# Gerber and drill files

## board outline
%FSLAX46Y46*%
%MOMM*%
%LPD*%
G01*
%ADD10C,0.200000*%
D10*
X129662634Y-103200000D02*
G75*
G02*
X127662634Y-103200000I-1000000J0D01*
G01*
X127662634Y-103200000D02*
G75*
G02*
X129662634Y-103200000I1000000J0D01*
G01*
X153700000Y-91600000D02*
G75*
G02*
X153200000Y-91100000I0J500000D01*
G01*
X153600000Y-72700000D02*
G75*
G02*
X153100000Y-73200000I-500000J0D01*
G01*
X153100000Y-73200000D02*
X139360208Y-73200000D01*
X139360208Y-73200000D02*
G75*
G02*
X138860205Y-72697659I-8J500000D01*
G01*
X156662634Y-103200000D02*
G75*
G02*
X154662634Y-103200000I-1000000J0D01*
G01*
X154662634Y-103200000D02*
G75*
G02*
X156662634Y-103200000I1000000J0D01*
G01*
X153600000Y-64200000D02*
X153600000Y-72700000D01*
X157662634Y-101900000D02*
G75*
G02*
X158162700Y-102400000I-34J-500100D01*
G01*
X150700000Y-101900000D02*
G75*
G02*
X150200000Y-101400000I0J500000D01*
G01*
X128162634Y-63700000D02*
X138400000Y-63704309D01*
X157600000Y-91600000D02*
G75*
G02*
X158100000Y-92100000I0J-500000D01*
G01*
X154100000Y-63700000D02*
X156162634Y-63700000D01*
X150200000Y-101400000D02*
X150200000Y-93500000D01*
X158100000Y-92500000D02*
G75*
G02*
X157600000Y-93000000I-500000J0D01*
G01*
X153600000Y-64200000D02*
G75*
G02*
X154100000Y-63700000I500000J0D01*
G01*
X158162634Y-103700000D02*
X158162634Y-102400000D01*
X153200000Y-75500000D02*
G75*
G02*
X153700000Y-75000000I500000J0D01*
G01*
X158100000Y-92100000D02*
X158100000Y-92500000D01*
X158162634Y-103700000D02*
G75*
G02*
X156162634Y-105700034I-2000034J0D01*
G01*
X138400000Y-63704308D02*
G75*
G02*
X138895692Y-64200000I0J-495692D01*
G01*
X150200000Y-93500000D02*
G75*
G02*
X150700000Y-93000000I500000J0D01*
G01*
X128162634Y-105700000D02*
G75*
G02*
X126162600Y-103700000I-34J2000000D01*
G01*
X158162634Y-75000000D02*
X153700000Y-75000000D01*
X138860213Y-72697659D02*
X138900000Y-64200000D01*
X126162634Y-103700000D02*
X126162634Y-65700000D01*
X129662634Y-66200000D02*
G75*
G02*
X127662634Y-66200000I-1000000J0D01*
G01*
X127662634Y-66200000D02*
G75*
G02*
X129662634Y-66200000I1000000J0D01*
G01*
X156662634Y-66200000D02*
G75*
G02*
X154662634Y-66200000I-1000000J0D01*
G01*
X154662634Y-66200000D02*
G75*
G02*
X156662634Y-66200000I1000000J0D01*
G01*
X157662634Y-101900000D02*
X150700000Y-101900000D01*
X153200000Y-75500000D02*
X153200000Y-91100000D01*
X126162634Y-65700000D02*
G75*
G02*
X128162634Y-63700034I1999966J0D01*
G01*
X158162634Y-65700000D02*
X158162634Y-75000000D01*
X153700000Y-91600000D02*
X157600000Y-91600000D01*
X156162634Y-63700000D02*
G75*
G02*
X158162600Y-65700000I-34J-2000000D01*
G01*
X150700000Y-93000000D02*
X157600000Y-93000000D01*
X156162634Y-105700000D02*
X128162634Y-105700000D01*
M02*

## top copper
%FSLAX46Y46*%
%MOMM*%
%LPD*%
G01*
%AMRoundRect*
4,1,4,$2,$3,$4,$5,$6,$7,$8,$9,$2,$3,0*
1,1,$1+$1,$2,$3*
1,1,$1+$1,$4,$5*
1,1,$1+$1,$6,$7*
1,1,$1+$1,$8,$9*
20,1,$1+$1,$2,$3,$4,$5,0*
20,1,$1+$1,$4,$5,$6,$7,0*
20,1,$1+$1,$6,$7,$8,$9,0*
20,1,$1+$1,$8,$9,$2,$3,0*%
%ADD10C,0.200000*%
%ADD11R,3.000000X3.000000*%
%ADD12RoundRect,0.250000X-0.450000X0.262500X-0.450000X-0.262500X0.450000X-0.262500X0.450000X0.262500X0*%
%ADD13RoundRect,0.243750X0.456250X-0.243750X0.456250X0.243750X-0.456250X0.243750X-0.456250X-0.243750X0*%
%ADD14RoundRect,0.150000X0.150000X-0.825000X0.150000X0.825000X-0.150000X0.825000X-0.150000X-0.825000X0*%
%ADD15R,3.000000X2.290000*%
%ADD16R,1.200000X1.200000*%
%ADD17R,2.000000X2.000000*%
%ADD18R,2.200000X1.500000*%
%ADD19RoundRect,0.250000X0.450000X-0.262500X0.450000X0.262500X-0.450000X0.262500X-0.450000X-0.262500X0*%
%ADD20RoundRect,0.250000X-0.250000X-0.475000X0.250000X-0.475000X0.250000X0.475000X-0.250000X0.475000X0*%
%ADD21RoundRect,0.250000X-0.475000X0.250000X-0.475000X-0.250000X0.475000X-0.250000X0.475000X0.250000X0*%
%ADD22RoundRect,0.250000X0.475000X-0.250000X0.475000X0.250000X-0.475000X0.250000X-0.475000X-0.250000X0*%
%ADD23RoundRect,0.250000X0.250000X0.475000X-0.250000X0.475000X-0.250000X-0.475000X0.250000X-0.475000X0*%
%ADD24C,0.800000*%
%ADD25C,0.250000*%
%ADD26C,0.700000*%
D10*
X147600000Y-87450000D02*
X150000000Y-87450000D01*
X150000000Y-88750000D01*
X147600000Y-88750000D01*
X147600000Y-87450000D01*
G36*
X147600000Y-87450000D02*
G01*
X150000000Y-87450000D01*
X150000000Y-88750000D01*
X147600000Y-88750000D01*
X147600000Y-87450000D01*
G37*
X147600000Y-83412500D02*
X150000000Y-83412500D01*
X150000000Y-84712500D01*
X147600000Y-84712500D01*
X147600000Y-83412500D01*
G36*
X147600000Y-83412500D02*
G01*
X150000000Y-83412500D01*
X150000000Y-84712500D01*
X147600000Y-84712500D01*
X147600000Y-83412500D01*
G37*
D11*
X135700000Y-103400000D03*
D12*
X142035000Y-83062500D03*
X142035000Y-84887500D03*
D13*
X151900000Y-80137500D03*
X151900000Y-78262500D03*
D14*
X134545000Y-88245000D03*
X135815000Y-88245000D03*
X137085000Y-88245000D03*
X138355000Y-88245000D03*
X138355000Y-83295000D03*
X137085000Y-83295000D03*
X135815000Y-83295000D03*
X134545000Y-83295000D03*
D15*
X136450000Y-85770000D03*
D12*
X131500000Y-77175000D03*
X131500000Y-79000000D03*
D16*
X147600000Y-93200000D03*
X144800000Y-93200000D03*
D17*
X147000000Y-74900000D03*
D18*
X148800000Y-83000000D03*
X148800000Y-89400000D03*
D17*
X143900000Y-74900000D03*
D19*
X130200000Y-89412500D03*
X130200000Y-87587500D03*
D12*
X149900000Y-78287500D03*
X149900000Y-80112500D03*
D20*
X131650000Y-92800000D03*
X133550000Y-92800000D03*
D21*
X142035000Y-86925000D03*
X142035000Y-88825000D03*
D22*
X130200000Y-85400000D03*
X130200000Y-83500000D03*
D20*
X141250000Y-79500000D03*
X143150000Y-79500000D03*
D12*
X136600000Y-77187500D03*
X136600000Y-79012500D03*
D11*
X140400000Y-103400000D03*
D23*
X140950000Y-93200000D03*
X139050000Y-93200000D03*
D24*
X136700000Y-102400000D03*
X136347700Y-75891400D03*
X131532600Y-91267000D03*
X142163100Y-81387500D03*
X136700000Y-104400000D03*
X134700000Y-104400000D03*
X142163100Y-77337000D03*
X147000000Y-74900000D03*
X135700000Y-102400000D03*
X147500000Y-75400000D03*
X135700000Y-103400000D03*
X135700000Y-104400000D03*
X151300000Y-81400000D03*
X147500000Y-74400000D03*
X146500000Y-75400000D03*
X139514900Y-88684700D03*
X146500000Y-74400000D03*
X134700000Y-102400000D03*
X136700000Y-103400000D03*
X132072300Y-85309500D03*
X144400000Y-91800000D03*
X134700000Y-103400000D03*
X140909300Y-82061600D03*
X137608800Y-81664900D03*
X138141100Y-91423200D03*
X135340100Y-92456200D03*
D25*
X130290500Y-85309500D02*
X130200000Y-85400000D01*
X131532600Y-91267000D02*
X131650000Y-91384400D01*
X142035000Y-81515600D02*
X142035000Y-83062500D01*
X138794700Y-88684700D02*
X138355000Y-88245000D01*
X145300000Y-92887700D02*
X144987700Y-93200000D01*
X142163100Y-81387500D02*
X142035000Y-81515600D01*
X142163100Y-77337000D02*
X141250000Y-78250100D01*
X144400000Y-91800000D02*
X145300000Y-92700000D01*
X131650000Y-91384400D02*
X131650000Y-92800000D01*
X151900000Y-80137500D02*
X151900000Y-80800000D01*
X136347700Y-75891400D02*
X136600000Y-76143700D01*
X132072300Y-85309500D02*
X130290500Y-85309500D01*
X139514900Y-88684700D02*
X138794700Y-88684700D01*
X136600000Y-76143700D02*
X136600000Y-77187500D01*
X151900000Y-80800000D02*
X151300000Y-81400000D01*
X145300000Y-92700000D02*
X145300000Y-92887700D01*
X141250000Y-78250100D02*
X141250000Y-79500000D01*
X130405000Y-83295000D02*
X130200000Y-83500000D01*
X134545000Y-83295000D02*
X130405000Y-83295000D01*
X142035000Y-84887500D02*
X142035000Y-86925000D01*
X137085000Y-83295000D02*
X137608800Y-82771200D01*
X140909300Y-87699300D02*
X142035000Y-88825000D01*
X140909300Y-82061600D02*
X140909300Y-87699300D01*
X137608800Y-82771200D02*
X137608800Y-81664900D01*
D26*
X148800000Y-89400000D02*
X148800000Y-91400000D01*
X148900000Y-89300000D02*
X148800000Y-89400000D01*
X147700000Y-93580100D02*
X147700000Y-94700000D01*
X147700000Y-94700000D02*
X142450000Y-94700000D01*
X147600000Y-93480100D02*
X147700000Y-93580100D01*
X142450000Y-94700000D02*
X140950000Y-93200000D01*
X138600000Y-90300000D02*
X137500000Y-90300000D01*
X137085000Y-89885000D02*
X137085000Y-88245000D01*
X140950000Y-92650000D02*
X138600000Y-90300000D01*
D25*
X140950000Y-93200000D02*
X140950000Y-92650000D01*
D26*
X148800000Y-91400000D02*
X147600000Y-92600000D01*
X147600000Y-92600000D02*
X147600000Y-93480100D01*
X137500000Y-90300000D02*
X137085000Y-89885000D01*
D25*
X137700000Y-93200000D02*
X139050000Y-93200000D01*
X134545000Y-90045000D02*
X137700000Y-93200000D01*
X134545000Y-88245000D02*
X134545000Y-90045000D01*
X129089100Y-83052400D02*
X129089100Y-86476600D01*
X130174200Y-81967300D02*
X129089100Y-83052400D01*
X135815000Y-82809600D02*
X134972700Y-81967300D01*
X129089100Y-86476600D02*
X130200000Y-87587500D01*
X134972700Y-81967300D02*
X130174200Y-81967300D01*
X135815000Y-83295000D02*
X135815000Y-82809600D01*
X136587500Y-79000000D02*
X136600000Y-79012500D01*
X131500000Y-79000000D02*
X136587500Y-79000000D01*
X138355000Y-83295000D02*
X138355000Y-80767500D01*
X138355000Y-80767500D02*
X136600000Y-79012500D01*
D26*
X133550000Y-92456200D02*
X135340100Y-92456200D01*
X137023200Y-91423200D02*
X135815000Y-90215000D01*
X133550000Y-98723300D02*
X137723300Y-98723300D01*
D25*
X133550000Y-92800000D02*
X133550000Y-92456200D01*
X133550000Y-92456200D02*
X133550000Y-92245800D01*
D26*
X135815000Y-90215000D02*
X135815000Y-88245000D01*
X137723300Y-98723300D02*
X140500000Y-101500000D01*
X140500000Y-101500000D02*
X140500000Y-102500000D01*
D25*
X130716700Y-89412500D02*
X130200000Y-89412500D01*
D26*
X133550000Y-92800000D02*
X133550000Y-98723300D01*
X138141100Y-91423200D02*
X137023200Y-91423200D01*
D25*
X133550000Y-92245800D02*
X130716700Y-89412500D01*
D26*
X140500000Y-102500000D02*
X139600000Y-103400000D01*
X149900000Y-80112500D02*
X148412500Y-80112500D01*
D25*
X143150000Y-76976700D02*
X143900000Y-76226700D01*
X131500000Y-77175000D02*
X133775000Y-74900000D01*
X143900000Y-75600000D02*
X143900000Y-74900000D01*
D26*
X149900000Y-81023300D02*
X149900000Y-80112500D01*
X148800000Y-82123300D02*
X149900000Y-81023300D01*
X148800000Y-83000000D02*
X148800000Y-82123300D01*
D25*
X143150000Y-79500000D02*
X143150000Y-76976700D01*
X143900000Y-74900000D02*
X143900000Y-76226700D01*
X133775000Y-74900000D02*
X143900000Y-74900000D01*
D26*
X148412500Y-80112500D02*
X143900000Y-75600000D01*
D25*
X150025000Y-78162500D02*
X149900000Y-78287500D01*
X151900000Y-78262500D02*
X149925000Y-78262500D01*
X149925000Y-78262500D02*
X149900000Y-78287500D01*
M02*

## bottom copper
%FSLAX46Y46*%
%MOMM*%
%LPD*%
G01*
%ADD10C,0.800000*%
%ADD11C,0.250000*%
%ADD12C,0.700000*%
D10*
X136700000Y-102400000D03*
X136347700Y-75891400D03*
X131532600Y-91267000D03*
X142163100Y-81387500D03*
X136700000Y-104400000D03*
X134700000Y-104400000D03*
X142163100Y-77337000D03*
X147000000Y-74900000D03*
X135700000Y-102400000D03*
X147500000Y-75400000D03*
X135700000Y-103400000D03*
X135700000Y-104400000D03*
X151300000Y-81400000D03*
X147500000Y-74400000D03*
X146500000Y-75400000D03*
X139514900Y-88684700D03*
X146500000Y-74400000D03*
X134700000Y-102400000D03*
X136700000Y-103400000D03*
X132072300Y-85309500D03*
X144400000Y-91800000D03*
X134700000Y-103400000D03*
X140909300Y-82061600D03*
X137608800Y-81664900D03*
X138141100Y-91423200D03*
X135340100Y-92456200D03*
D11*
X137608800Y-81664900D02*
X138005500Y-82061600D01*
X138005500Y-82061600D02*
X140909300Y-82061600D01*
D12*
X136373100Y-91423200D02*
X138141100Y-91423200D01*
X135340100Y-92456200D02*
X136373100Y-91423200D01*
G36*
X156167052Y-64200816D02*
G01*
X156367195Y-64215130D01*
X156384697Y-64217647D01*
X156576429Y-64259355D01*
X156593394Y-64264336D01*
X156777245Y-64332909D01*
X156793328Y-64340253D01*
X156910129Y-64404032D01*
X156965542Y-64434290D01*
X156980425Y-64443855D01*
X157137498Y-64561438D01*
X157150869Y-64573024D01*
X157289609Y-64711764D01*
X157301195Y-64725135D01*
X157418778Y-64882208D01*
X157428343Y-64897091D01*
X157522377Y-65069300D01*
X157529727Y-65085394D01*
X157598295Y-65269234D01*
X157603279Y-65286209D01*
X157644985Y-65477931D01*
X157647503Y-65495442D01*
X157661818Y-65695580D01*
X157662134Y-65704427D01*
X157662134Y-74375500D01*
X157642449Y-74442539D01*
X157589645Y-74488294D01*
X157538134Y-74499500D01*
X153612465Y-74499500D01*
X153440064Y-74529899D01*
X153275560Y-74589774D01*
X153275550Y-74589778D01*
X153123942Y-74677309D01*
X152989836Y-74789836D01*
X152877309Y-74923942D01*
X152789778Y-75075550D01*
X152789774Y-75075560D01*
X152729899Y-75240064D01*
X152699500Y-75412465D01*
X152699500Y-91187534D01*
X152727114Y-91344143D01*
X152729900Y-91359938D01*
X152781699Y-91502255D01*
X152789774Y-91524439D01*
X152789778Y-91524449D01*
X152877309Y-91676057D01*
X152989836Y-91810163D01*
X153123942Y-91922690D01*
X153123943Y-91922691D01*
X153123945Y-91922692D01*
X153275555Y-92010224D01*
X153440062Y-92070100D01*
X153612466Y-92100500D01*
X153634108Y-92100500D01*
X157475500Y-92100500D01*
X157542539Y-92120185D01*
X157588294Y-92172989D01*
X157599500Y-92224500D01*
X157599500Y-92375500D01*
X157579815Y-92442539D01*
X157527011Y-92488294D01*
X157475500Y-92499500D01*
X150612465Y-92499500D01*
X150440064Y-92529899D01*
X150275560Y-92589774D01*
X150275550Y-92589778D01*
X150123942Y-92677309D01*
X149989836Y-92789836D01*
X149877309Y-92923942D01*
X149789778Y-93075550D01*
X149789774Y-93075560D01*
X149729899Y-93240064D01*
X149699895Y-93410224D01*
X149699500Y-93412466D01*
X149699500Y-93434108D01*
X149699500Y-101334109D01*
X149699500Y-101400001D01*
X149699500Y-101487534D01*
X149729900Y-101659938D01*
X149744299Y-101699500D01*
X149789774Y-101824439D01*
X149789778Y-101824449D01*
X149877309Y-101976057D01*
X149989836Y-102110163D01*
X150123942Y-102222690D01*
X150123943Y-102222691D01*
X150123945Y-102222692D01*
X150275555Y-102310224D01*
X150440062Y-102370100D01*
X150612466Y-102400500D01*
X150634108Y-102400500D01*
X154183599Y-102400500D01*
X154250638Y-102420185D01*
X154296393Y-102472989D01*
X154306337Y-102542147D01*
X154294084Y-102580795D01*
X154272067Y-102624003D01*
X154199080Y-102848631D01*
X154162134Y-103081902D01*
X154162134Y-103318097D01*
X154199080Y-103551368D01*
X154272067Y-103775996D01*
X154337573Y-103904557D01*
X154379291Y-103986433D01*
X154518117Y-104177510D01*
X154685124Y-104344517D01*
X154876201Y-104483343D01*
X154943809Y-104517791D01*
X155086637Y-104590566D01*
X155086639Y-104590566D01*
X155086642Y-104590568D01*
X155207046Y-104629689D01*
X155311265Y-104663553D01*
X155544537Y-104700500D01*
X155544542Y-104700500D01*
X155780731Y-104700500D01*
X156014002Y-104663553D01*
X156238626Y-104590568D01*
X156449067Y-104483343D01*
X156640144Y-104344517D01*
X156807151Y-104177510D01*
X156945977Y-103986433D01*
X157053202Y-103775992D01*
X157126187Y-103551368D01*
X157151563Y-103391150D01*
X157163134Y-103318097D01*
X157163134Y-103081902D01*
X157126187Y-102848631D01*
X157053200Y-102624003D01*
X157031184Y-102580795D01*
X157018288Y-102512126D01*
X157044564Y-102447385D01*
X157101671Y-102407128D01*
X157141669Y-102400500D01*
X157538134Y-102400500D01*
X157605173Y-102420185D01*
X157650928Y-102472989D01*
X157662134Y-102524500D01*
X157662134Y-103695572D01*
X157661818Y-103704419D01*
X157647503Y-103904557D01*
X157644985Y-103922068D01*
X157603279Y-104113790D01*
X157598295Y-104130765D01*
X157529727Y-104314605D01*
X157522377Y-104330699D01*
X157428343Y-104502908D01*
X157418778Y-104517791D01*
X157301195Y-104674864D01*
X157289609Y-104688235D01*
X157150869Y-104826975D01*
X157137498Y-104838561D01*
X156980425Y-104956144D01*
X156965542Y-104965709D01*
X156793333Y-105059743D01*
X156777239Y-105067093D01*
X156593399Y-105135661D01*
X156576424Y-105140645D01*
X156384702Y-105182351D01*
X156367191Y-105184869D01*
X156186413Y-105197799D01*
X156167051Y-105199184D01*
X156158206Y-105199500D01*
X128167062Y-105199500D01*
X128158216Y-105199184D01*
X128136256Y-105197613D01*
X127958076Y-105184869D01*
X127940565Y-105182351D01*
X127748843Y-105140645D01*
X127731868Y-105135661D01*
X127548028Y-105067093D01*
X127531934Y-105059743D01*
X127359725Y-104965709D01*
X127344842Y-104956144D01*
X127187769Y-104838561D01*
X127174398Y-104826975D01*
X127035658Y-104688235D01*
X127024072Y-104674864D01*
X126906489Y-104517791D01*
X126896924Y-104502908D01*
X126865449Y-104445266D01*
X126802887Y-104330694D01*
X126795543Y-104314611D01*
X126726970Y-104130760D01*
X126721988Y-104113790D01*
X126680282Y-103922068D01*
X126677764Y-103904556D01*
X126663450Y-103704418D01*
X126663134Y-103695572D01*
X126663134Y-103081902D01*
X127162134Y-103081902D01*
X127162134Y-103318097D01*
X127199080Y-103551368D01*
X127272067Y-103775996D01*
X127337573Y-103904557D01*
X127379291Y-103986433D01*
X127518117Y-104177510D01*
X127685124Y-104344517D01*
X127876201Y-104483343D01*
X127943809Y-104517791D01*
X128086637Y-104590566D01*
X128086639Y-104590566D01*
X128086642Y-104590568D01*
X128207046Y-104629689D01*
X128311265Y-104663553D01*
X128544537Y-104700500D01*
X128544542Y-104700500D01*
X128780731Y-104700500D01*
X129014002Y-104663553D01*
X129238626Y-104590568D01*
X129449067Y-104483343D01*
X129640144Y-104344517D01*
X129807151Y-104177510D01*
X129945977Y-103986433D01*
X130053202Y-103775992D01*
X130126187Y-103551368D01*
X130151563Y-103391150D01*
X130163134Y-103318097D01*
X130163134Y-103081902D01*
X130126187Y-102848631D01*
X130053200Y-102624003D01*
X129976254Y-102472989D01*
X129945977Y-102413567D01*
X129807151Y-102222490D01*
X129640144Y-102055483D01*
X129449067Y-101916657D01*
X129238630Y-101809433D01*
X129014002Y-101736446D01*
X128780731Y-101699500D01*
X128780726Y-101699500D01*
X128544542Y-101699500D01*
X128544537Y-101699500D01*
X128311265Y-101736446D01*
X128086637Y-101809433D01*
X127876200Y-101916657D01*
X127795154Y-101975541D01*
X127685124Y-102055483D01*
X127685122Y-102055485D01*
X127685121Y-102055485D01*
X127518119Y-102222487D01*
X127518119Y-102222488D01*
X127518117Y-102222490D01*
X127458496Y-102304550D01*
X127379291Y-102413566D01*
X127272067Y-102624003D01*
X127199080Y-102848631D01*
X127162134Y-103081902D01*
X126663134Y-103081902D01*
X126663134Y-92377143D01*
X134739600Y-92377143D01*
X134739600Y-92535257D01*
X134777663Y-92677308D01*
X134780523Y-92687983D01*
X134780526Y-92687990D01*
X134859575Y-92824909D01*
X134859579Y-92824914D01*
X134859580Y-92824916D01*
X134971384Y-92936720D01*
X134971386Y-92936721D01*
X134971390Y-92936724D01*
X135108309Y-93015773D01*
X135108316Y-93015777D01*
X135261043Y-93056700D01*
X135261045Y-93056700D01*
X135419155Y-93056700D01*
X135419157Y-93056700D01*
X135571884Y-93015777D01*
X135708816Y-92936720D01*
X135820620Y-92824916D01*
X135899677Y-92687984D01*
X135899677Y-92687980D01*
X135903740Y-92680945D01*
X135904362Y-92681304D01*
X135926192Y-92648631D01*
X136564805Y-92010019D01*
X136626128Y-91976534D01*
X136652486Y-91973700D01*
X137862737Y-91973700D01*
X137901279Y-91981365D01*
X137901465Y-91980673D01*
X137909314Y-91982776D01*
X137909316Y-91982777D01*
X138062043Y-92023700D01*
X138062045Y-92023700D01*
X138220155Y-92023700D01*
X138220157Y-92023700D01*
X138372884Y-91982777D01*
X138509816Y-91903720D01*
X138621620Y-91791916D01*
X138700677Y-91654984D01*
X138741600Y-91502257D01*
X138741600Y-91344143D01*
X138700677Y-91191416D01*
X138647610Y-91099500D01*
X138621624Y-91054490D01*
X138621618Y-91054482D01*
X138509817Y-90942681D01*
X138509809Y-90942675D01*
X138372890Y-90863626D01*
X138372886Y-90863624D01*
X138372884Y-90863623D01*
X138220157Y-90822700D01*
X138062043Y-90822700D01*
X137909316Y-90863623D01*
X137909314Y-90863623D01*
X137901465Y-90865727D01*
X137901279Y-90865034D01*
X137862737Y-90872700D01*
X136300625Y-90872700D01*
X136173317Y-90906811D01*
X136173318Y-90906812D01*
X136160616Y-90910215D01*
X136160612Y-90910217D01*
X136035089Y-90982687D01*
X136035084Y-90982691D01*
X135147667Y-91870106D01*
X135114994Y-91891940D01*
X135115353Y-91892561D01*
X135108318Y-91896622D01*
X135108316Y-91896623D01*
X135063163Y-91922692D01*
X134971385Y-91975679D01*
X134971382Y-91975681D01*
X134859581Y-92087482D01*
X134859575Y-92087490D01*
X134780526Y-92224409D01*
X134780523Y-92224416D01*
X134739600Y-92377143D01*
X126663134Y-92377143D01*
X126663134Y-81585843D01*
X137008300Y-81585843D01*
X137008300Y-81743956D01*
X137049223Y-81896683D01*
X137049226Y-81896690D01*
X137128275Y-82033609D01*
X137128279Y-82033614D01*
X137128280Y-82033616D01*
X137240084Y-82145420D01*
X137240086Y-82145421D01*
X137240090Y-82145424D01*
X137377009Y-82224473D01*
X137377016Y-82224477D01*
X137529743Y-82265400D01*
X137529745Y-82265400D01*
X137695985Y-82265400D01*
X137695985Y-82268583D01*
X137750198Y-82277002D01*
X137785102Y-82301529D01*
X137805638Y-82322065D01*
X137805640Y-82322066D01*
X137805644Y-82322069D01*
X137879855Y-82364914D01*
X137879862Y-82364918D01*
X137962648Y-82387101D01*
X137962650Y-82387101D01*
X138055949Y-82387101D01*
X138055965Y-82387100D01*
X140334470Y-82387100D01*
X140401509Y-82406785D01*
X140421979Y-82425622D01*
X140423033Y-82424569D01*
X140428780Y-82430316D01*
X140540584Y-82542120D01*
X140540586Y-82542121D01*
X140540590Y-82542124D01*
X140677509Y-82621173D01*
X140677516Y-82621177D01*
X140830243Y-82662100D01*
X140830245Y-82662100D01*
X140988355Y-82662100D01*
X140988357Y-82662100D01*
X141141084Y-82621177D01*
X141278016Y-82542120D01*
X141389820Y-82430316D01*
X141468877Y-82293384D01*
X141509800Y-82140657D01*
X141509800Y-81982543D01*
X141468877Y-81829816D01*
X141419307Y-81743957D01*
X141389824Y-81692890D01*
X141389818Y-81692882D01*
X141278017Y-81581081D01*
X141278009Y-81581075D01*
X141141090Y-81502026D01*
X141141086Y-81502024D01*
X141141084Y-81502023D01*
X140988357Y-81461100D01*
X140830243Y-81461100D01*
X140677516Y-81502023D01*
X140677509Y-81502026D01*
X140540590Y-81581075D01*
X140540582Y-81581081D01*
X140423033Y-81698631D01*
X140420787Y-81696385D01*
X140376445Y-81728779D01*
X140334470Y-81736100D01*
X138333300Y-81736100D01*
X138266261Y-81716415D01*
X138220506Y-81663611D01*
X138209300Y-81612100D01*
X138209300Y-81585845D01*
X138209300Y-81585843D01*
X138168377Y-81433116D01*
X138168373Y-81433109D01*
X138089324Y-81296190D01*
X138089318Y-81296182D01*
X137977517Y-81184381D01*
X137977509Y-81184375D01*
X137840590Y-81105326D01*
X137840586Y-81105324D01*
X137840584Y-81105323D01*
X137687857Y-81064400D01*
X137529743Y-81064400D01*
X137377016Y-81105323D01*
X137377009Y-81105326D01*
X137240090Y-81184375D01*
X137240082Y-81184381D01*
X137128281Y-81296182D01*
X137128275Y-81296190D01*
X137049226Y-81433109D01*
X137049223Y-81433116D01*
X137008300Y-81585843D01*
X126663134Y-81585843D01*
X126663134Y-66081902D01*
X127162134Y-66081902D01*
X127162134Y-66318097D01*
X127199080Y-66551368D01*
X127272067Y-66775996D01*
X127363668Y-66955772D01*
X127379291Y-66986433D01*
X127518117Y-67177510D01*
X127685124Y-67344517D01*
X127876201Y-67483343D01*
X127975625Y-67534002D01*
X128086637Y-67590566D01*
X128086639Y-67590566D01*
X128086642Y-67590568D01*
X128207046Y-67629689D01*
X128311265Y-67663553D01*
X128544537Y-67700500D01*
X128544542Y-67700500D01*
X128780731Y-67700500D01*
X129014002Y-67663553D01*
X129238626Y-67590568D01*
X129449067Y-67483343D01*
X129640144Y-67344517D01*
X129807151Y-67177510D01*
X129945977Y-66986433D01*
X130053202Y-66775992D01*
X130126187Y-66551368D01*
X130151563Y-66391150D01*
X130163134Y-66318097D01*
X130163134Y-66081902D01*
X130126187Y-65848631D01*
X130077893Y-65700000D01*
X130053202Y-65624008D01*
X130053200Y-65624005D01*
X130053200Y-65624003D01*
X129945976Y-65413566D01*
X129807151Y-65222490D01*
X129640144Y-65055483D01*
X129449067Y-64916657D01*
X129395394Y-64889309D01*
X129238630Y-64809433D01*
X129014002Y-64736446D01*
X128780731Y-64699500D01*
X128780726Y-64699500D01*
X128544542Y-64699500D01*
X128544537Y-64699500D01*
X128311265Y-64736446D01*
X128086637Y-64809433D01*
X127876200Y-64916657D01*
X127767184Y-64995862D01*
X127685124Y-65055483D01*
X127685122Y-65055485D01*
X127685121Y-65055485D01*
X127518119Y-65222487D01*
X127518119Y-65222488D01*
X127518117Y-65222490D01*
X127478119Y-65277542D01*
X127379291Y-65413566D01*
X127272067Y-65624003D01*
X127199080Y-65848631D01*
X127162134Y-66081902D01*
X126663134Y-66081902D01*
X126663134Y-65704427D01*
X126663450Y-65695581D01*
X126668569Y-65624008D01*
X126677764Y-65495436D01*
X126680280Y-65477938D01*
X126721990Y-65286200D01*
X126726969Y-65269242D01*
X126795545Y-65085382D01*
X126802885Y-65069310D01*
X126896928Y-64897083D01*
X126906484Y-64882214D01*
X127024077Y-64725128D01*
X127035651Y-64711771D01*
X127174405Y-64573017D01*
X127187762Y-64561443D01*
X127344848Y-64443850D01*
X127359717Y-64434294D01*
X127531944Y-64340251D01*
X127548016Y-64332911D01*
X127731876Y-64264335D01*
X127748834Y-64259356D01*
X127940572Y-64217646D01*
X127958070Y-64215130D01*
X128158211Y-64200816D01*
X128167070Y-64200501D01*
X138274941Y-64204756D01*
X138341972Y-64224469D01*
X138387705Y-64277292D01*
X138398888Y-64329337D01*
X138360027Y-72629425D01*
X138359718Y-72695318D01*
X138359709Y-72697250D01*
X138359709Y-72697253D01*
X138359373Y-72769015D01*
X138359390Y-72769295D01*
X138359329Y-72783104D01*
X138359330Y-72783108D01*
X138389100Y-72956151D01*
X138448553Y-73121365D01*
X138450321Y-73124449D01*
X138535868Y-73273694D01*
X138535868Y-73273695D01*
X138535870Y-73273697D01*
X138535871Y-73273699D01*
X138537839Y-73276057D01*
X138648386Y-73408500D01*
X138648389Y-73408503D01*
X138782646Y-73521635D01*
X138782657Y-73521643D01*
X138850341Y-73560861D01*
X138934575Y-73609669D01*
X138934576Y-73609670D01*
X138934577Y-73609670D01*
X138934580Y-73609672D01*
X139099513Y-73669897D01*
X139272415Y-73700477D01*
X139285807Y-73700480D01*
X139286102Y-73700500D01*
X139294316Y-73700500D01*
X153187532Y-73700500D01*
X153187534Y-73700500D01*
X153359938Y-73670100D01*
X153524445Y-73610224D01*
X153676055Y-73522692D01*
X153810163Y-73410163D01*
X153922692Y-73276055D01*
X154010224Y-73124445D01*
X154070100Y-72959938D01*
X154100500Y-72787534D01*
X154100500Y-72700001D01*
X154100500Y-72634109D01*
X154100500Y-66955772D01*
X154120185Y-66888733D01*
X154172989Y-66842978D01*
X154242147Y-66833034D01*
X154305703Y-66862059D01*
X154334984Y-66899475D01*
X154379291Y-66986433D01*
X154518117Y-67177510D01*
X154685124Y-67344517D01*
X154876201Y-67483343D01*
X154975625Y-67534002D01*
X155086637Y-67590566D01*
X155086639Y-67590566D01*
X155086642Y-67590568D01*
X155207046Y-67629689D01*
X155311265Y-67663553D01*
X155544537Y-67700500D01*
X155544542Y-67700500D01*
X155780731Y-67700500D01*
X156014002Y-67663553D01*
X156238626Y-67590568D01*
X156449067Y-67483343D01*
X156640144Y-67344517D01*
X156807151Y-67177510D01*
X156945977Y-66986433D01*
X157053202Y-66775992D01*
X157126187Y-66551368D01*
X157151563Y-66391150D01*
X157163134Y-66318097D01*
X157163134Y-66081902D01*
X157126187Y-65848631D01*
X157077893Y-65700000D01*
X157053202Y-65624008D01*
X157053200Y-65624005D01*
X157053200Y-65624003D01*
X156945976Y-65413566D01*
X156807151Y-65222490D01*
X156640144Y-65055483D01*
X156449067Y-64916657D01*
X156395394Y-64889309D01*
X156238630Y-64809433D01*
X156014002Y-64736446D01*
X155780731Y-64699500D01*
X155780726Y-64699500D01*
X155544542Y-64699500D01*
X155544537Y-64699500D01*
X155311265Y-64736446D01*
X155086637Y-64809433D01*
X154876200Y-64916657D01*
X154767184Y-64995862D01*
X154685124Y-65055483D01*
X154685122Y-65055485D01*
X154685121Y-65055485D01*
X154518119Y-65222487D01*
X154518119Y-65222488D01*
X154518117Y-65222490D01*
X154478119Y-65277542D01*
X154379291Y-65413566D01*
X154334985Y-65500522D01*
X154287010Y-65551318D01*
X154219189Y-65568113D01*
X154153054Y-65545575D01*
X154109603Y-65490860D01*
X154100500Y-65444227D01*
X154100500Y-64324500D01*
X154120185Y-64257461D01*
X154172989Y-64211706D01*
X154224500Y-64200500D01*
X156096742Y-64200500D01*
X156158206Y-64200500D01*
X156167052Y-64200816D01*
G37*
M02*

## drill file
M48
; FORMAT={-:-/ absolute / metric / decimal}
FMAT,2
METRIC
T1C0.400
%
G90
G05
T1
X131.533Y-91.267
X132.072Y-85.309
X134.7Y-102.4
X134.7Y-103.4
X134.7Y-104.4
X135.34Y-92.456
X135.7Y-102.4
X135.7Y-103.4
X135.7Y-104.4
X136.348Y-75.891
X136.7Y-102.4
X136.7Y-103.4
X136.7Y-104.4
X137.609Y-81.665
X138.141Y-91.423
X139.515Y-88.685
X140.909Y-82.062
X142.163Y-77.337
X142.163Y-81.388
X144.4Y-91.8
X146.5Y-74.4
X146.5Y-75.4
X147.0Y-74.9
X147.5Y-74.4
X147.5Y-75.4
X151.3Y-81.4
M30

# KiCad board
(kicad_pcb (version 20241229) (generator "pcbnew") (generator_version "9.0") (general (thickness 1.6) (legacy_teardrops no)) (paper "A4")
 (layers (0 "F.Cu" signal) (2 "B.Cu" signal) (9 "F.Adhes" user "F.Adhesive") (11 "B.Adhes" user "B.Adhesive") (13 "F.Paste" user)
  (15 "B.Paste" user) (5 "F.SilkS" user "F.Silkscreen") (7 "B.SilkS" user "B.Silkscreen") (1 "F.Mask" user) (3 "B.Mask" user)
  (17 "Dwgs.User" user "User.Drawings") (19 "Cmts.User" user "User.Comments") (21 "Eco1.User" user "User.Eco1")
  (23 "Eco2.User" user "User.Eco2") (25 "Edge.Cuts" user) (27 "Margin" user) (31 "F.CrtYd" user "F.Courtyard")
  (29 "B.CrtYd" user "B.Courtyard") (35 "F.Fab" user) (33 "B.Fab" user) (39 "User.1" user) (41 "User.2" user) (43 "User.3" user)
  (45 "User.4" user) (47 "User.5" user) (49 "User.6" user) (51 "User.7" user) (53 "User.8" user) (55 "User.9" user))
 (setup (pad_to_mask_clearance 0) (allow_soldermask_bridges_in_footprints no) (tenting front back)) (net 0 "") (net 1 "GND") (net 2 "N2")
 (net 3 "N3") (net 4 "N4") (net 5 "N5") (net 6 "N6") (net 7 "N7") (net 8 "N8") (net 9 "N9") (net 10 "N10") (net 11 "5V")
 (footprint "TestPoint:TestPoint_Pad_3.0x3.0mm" (layer "F.Cu") (at 135.7 103.4)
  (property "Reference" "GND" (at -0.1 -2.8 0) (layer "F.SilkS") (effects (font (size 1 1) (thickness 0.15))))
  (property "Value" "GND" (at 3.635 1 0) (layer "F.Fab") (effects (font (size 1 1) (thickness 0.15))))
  (pad "1" smd rect (at 0 0) (size 3 3) (layers "F.Cu" "F.Mask") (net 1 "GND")))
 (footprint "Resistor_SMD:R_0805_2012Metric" (layer "F.Cu") (at 142.035 83.975 -90)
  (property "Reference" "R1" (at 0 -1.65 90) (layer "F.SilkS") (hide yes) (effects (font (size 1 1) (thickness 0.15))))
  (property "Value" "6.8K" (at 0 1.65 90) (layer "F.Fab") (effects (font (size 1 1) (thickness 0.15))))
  (pad "1" smd roundrect (at -0.9125 0 270) (size 1.025 1.4) (layers "F.Cu" "F.Mask" "F.Paste") (roundrect_rratio 0.243902) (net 1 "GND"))
  (pad "2" smd roundrect (at 0.9125 0 270) (size 1.025 1.4) (layers "F.Cu" "F.Mask" "F.Paste") (roundrect_rratio 0.243902) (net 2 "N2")))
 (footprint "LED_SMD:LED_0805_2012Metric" (layer "F.Cu") (at 151.9 79.2 90)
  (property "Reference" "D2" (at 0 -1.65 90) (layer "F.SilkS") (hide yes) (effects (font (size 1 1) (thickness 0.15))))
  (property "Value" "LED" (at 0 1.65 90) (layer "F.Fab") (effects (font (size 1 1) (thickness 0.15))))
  (pad "1" smd roundrect (at -0.9375 0 90) (size 0.975 1.4) (layers "F.Cu" "F.Mask" "F.Paste") (roundrect_rratio 0.25) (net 1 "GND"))
  (pad "2" smd roundrect (at 0.9375 0 90) (size 0.975 1.4) (layers "F.Cu" "F.Mask" "F.Paste") (roundrect_rratio 0.25) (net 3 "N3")))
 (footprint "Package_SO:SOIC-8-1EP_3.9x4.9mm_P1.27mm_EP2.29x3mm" (layer "F.Cu") (at 136.45 85.77 90)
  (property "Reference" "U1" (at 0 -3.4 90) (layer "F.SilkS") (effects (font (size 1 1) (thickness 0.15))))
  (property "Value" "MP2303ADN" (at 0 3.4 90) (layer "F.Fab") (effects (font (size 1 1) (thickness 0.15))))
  (pad "" smd roundrect (at -0.57 -0.75 90) (size 0.92 1.21) (layers "F.Paste") (roundrect_rratio 0.25))
  (pad "" smd roundrect (at -0.57 0.75 90) (size 0.92 1.21) (layers "F.Paste") (roundrect_rratio 0.25))
  (pad "" smd roundrect (at 0.57 -0.75 90) (size 0.92 1.21) (layers "F.Paste") (roundrect_rratio 0.25))
  (pad "" smd roundrect (at 0.57 0.75 90) (size 0.92 1.21) (layers "F.Paste") (roundrect_rratio 0.25))
  (pad "1" smd roundrect (at -2.475 -1.905 90) (size 1.95 0.6) (layers "F.Cu" "F.Mask" "F.Paste") (roundrect_rratio 0.25) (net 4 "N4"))
  (pad "2" smd roundrect (at -2.475 -0.635 90) (size 1.95 0.6) (layers "F.Cu" "F.Mask" "F.Paste") (roundrect_rratio 0.25) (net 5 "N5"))
  (pad "3" smd roundrect (at -2.475 0.635 90) (size 1.95 0.6) (layers "F.Cu" "F.Mask" "F.Paste") (roundrect_rratio 0.25) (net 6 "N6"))
  (pad "4" smd roundrect (at -2.475 1.905 90) (size 1.95 0.6) (layers "F.Cu" "F.Mask" "F.Paste") (roundrect_rratio 0.25) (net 1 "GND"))
  (pad "5" smd roundrect (at 2.475 1.905 90) (size 1.95 0.6) (layers "F.Cu" "F.Mask" "F.Paste") (roundrect_rratio 0.25) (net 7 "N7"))
  (pad "6" smd roundrect (at 2.475 0.635 90) (size 1.95 0.6) (layers "F.Cu" "F.Mask" "F.Paste") (roundrect_rratio 0.25) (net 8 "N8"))
  (pad "7" smd roundrect (at 2.475 -0.635 90) (size 1.95 0.6) (layers "F.Cu" "F.Mask" "F.Paste") (roundrect_rratio 0.25) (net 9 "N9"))
  (pad "8" smd roundrect (at 2.475 -1.905 90) (size 1.95 0.6) (layers "F.Cu" "F.Mask" "F.Paste") (roundrect_rratio 0.25) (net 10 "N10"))
  (pad "9" smd rect (at 0 0 90) (size 2.29 3) (layers "F.Cu" "F.Mask") (zone_connect 2)))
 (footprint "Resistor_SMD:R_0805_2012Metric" (layer "F.Cu") (at 131.5 78.0875 -90)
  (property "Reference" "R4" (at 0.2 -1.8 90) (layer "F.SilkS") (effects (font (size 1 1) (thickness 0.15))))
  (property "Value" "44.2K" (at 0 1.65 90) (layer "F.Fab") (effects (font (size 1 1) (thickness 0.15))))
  (pad "1" smd roundrect (at -0.9125 0 270) (size 1.025 1.4) (layers "F.Cu" "F.Mask" "F.Paste") (roundrect_rratio 0.243902) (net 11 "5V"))
  (pad "2" smd roundrect (at 0.9125 0 270) (size 1.025 1.4) (layers "F.Cu" "F.Mask" "F.Paste") (roundrect_rratio 0.243902) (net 7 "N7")))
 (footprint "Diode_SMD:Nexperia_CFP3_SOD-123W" (layer "F.Cu") (at 146.2 93.2 180)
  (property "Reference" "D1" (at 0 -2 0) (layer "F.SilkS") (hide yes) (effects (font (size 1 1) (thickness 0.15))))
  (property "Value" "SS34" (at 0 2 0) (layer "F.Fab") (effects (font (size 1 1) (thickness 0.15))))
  (pad "1" smd rect (at -1.4 0 180) (size 1.2 1.2) (layers "F.Cu" "F.Mask" "F.Paste") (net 6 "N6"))
  (pad "2" smd rect (at 1.4 0 180) (size 1.2 1.2) (layers "F.Cu" "F.Mask" "F.Paste") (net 1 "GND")))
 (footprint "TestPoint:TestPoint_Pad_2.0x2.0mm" (layer "F.Cu") (at 147 74.9)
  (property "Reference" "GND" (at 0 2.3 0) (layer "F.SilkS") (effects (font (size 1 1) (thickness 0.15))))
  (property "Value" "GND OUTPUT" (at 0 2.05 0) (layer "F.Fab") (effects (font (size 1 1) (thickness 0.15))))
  (pad "1" smd rect (at 0 0) (size 2 2) (layers "F.Cu" "F.Mask") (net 1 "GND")))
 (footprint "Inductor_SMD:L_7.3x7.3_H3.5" (layer "F.Cu") (at 148.8 86.2 -90)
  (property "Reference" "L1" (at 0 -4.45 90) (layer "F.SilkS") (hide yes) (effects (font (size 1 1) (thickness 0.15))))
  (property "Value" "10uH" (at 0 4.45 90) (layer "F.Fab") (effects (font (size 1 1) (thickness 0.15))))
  (pad "1" smd rect (at -3.2 0 270) (size 1.5 2.2) (layers "F.Cu" "F.Mask" "F.Paste") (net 11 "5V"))
  (pad "2" smd rect (at 3.2 0 270) (size 1.5 2.2) (layers "F.Cu" "F.Mask" "F.Paste") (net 6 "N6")))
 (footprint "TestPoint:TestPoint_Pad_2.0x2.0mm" (layer "F.Cu") (at 143.9 74.9)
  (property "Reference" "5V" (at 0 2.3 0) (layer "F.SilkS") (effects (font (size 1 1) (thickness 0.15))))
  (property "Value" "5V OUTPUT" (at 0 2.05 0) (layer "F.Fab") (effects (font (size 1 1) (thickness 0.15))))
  (pad "1" smd rect (at 0 0) (size 2 2) (layers "F.Cu" "F.Mask") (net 11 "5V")))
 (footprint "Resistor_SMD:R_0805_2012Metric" (layer "F.Cu") (at 130.2 88.5 90)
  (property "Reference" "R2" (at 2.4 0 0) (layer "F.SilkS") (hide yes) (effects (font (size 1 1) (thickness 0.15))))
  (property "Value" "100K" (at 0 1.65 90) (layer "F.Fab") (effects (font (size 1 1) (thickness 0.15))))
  (pad "1" smd roundrect (at -0.9125 0 90) (size 1.025 1.4) (layers "F.Cu" "F.Mask" "F.Paste") (roundrect_rratio 0.243902) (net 5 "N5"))
  (pad "2" smd roundrect (at 0.9125 0 90) (size 1.025 1.4) (layers "F.Cu" "F.Mask" "F.Paste") (roundrect_rratio 0.243902) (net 9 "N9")))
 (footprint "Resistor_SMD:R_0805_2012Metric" (layer "F.Cu") (at 149.9 79.2 -90)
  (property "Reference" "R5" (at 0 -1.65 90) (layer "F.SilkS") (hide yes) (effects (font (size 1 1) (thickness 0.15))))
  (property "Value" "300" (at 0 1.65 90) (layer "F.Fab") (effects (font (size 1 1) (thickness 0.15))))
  (pad "1" smd roundrect (at -0.9125 0 270) (size 1.025 1.4) (layers "F.Cu" "F.Mask" "F.Paste") (roundrect_rratio 0.243902) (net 3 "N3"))
  (pad "2" smd roundrect (at 0.9125 0 270) (size 1.025 1.4) (layers "F.Cu" "F.Mask" "F.Paste") (roundrect_rratio 0.243902) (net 11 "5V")))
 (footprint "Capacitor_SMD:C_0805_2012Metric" (layer "F.Cu") (at 132.6 92.8)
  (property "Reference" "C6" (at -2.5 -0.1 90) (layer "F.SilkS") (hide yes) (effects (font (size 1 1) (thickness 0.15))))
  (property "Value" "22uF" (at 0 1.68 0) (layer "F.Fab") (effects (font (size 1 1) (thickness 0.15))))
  (pad "1" smd roundrect (at -0.95 0) (size 1 1.45) (layers "F.Cu" "F.Mask" "F.Paste") (roundrect_rratio 0.25) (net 1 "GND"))
  (pad "2" smd roundrect (at 0.95 0) (size 1 1.45) (layers "F.Cu" "F.Mask" "F.Paste") (roundrect_rratio 0.25) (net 5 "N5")))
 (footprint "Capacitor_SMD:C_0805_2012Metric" (layer "F.Cu") (at 142.035 87.875 -90)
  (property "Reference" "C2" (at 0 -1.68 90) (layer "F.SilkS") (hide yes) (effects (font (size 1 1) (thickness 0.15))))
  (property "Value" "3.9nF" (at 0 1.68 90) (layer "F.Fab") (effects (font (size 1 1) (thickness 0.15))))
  (pad "1" smd roundrect (at -0.95 0 270) (size 1 1.45) (layers "F.Cu" "F.Mask" "F.Paste") (roundrect_rratio 0.25) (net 2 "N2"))
  (pad "2" smd roundrect (at 0.95 0 270) (size 1 1.45) (layers "F.Cu" "F.Mask" "F.Paste") (roundrect_rratio 0.25) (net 8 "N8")))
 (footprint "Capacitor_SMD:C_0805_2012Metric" (layer "F.Cu") (at 130.2 84.45 90)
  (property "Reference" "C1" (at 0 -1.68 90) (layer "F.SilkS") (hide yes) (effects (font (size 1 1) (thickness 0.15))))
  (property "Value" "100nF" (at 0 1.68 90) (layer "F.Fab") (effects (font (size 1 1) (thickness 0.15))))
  (pad "1" smd roundrect (at -0.95 0 90) (size 1 1.45) (layers "F.Cu" "F.Mask" "F.Paste") (roundrect_rratio 0.25) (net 1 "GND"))
  (pad "2" smd roundrect (at 0.95 0 90) (size 1 1.45) (layers "F.Cu" "F.Mask" "F.Paste") (roundrect_rratio 0.25) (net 10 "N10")))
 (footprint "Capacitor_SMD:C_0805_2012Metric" (layer "F.Cu") (at 142.2 79.5)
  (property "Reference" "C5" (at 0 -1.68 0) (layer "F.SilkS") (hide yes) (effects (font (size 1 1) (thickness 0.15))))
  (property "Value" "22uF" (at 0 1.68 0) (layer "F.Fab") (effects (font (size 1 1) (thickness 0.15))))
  (pad "1" smd roundrect (at -0.95 0) (size 1 1.45) (layers "F.Cu" "F.Mask" "F.Paste") (roundrect_rratio 0.25) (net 1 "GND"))
  (pad "2" smd roundrect (at 0.95 0) (size 1 1.45) (layers "F.Cu" "F.Mask" "F.Paste") (roundrect_rratio 0.25) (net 11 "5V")))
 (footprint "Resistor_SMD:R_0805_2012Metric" (layer "F.Cu") (at 136.6 78.1 -90)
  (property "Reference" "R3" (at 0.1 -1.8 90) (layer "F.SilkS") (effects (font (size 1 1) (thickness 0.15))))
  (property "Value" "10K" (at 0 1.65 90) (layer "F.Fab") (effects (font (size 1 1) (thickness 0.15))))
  (pad "1" smd roundrect (at -0.9125 0 270) (size 1.025 1.4) (layers "F.Cu" "F.Mask" "F.Paste") (roundrect_rratio 0.243902) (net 1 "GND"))
  (pad "2" smd roundrect (at 0.9125 0 270) (size 1.025 1.4) (layers "F.Cu" "F.Mask" "F.Paste") (roundrect_rratio 0.243902) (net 7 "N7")))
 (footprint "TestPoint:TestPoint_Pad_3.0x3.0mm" (layer "F.Cu") (at 140.4 103.4)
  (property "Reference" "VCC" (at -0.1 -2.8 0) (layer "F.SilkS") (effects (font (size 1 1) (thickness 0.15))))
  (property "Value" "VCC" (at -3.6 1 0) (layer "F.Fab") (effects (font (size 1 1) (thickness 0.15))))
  (pad "1" smd rect (at 0 0) (size 3 3) (layers "F.Cu" "F.Mask") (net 5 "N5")))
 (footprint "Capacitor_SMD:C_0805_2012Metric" (layer "F.Cu") (at 140 93.2 180)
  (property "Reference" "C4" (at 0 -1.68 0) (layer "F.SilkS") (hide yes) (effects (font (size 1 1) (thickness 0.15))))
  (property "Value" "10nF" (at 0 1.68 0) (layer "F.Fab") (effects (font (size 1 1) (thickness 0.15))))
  (pad "1" smd roundrect (at -0.95 0 180) (size 1 1.45) (layers "F.Cu" "F.Mask" "F.Paste") (roundrect_rratio 0.25) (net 6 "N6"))
  (pad "2" smd roundrect (at 0.95 0 180) (size 1 1.45) (layers "F.Cu" "F.Mask" "F.Paste") (roundrect_rratio 0.25) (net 4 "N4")))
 (gr_rect (start 147.6 87.45) (end 150 88.75) (stroke (width 0.2) (type solid)) (fill yes) (layer "F.Cu") (net 6))
 (gr_rect (start 147.6 83.4125) (end 150 84.7125) (stroke (width 0.2) (type solid)) (fill yes) (layer "F.Cu") (net 11))
 (gr_circle (center 128.662634 103.2) (end 127.662634 103.2) (stroke (width 0.2) (type solid)) (fill no) (layer "Edge.Cuts"))
 (gr_arc (start 153.7 91.6) (mid 153.346447 91.453553) (end 153.2 91.1) (stroke (width 0.2) (type default)) (layer "Edge.Cuts"))
 (gr_arc (start 153.6 72.7) (mid 153.453553 73.053553) (end 153.1 73.2) (stroke (width 0.2) (type default)) (layer "Edge.Cuts"))
 (gr_line (start 153.1 73.2) (end 139.360208 73.2) (stroke (width 0.2) (type default)) (layer "Edge.Cuts"))
 (gr_arc (start 139.360208 73.2) (mid 139.005828 73.052725) (end 138.860213 72.697659) (stroke (width 0.2) (type default))
  (layer "Edge.Cuts"))
 (gr_circle (center 155.662634 103.2) (end 154.662634 103.2) (stroke (width 0.2) (type solid)) (fill no) (layer "Edge.Cuts"))
 (gr_line (start 153.6 64.2) (end 153.6 72.7) (stroke (width 0.2) (type default)) (layer "Edge.Cuts"))
 (gr_arc (start 157.662634 101.9) (mid 158.016165 102.046459) (end 158.162634 102.4) (stroke (width 0.2) (type default)) (layer "Edge.Cuts"))
 (gr_arc (start 150.7 101.9) (mid 150.346447 101.753553) (end 150.2 101.4) (stroke (width 0.2) (type default)) (layer "Edge.Cuts"))
 (gr_line (start 128.162634 63.7) (end 138.4 63.704309) (stroke (width 0.2) (type solid)) (layer "Edge.Cuts"))
 (gr_arc (start 157.6 91.6) (mid 157.953553 91.746447) (end 158.1 92.1) (stroke (width 0.2) (type default)) (layer "Edge.Cuts"))
 (gr_line (start 154.1 63.7) (end 156.162634 63.7) (stroke (width 0.2) (type default)) (layer "Edge.Cuts"))
 (gr_line (start 150.2 101.4) (end 150.2 93.5) (stroke (width 0.2) (type solid)) (layer "Edge.Cuts"))
 (gr_arc (start 158.1 92.5) (mid 157.953553 92.853553) (end 157.6 93) (stroke (width 0.2) (type default)) (layer "Edge.Cuts"))
 (gr_arc (start 153.6 64.2) (mid 153.746447 63.846447) (end 154.1 63.7) (stroke (width 0.2) (type default)) (layer "Edge.Cuts"))
 (gr_line (start 158.162634 103.7) (end 158.162634 102.4) (stroke (width 0.2) (type solid)) (layer "Edge.Cuts"))
 (gr_arc (start 153.2 75.5) (mid 153.346447 75.146447) (end 153.7 75) (stroke (width 0.2) (type default)) (layer "Edge.Cuts"))
 (gr_line (start 158.1 92.1) (end 158.1 92.5) (stroke (width 0.2) (type solid)) (layer "Edge.Cuts"))
 (gr_arc (start 158.162634 103.7) (mid 157.576848 105.114214) (end 156.162634 105.7) (stroke (width 0.2) (type solid)) (layer "Edge.Cuts"))
 (gr_arc (start 138.4 63.704308) (mid 138.750507 63.849493) (end 138.895692 64.2) (stroke (width 0.2) (type default)) (layer "Edge.Cuts"))
 (gr_arc (start 150.2 93.5) (mid 150.346447 93.146447) (end 150.7 93) (stroke (width 0.2) (type default)) (layer "Edge.Cuts"))
 (gr_arc (start 128.162634 105.7) (mid 126.74842 105.114214) (end 126.162634 103.7) (stroke (width 0.2) (type solid)) (layer "Edge.Cuts"))
 (gr_line (start 158.162634 75) (end 153.7 75) (stroke (width 0.2) (type solid)) (layer "Edge.Cuts"))
 (gr_line (start 138.860213 72.697659) (end 138.9 64.2) (stroke (width 0.2) (type default)) (layer "Edge.Cuts"))
 (gr_line (start 126.162634 103.7) (end 126.162634 65.7) (stroke (width 0.2) (type solid)) (layer "Edge.Cuts"))
 (gr_circle (center 128.662634 66.2) (end 127.662634 66.2) (stroke (width 0.2) (type solid)) (fill no) (layer "Edge.Cuts"))
 (gr_circle (center 155.662634 66.2) (end 154.662634 66.2) (stroke (width 0.2) (type solid)) (fill no) (layer "Edge.Cuts"))
 (gr_line (start 157.662634 101.9) (end 150.7 101.9) (stroke (width 0.2) (type solid)) (layer "Edge.Cuts"))
 (gr_line (start 153.2 75.5) (end 153.2 91.1) (stroke (width 0.2) (type solid)) (layer "Edge.Cuts"))
 (gr_arc (start 126.162634 65.7) (mid 126.74842 64.285786) (end 128.162634 63.7) (stroke (width 0.2) (type solid)) (layer "Edge.Cuts"))
 (gr_line (start 158.162634 65.7) (end 158.162634 75) (stroke (width 0.2) (type solid)) (layer "Edge.Cuts"))
 (gr_line (start 153.7 91.6) (end 157.6 91.6) (stroke (width 0.2) (type solid)) (layer "Edge.Cuts"))
 (gr_arc (start 156.162634 63.7) (mid 157.576848 64.285786) (end 158.162634 65.7) (stroke (width 0.2) (type solid)) (layer "Edge.Cuts"))
 (gr_line (start 150.7 93) (end 157.6 93) (stroke (width 0.2) (type solid)) (layer "Edge.Cuts"))
 (gr_line (start 156.162634 105.7) (end 128.162634 105.7) (stroke (width 0.2) (type solid)) (layer "Edge.Cuts"))
 (segment (start 130.2905 85.3095) (end 130.2 85.4) (width 0.25) (layer "F.Cu") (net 1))
 (segment (start 131.5326 91.267) (end 131.65 91.3844) (width 0.25) (layer "F.Cu") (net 1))
 (segment (start 142.035 81.5156) (end 142.035 83.0625) (width 0.25) (layer "F.Cu") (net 1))
 (segment (start 138.7947 88.6847) (end 138.355 88.245) (width 0.25) (layer "F.Cu") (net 1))
 (segment (start 145.3 92.8877) (end 144.9877 93.2) (width 0.25) (layer "F.Cu") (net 1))
 (segment (start 142.1631 81.3875) (end 142.035 81.5156) (width 0.25) (layer "F.Cu") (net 1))
 (segment (start 142.1631 77.337) (end 141.25 78.2501) (width 0.25) (layer "F.Cu") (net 1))
 (segment (start 144.4 91.8) (end 145.3 92.7) (width 0.25) (layer "F.Cu") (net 1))
 (segment (start 131.65 91.3844) (end 131.65 92.8) (width 0.25) (layer "F.Cu") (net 1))
 (segment (start 151.9 80.1375) (end 151.9 80.8) (width 0.25) (layer "F.Cu") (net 1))
 (segment (start 136.3477 75.8914) (end 136.6 76.1437) (width 0.25) (layer "F.Cu") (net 1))
 (segment (start 132.0723 85.3095) (end 130.2905 85.3095) (width 0.25) (layer "F.Cu") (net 1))
 (segment (start 139.5149 88.6847) (end 138.7947 88.6847) (width 0.25) (layer "F.Cu") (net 1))
 (segment (start 136.6 76.1437) (end 136.6 77.1875) (width 0.25) (layer "F.Cu") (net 1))
 (segment (start 151.9 80.8) (end 151.3 81.4) (width 0.25) (layer "F.Cu") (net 1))
 (segment (start 145.3 92.7) (end 145.3 92.8877) (width 0.25) (layer "F.Cu") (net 1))
 (segment (start 141.25 78.2501) (end 141.25 79.5) (width 0.25) (layer "F.Cu") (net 1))
 (via (at 136.7 102.4) (size 0.8) (drill 0.4) (layers "F.Cu" "B.Cu") (free yes) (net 1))
 (via (at 136.3477 75.8914) (size 0.8) (drill 0.4) (layers "F.Cu" "B.Cu") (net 1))
 (via (at 131.5326 91.267) (size 0.8) (drill 0.4) (layers "F.Cu" "B.Cu") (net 1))
 (via (at 142.1631 81.3875) (size 0.8) (drill 0.4) (layers "F.Cu" "B.Cu") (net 1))
 (via (at 136.7 104.4) (size 0.8) (drill 0.4) (layers "F.Cu" "B.Cu") (free yes) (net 1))
 (via (at 134.7 104.4) (size 0.8) (drill 0.4) (layers "F.Cu" "B.Cu") (free yes) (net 1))
 (via (at 142.1631 77.337) (size 0.8) (drill 0.4) (layers "F.Cu" "B.Cu") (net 1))
 (via (at 147 74.9) (size 0.8) (drill 0.4) (layers "F.Cu" "B.Cu") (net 1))
 (via (at 135.7 102.4) (size 0.8) (drill 0.4) (layers "F.Cu" "B.Cu") (free yes) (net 1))
 (via (at 147.5 75.4) (size 0.8) (drill 0.4) (layers "F.Cu" "B.Cu") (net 1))
 (via (at 135.7 103.4) (size 0.8) (drill 0.4) (layers "F.Cu" "B.Cu") (free yes) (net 1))
 (via (at 135.7 104.4) (size 0.8) (drill 0.4) (layers "F.Cu" "B.Cu") (free yes) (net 1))
 (via (at 151.3 81.4) (size 0.8) (drill 0.4) (layers "F.Cu" "B.Cu") (free yes) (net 1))
 (via (at 147.5 74.4) (size 0.8) (drill 0.4) (layers "F.Cu" "B.Cu") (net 1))
 (via (at 146.5 75.4) (size 0.8) (drill 0.4) (layers "F.Cu" "B.Cu") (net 1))
 (via (at 139.5149 88.6847) (size 0.8) (drill 0.4) (layers "F.Cu" "B.Cu") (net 1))
 (via (at 146.5 74.4) (size 0.8) (drill 0.4) (layers "F.Cu" "B.Cu") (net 1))
 (via (at 134.7 102.4) (size 0.8) (drill 0.4) (layers "F.Cu" "B.Cu") (free yes) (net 1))
 (via (at 136.7 103.4) (size 0.8) (drill 0.4) (layers "F.Cu" "B.Cu") (free yes) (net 1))
 (via (at 132.0723 85.3095) (size 0.8) (drill 0.4) (layers "F.Cu" "B.Cu") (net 1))
 (via (at 144.4 91.8) (size 0.8) (drill 0.4) (layers "F.Cu" "B.Cu") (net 1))
 (via (at 134.7 103.4) (size 0.8) (drill 0.4) (layers "F.Cu" "B.Cu") (free yes) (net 1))
 (segment (start 130.405 83.295) (end 130.2 83.5) (width 0.25) (layer "F.Cu") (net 10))
 (segment (start 134.545 83.295) (end 130.405 83.295) (width 0.25) (layer "F.Cu") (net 10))
 (segment (start 142.035 84.8875) (end 142.035 86.925) (width 0.25) (layer "F.Cu") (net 2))
 (segment (start 137.085 83.295) (end 137.6088 82.7712) (width 0.25) (layer "F.Cu") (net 8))
 (segment (start 140.9093 87.6993) (end 142.035 88.825) (width 0.25) (layer "F.Cu") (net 8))
 (segment (start 140.9093 82.0616) (end 140.9093 87.6993) (width 0.25) (layer "F.Cu") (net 8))
 (segment (start 137.6088 82.7712) (end 137.6088 81.6649) (width 0.25) (layer "F.Cu") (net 8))
 (via (at 140.9093 82.0616) (size 0.8) (drill 0.4) (layers "F.Cu" "B.Cu") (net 8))
 (via (at 137.6088 81.6649) (size 0.8) (drill 0.4) (layers "F.Cu" "B.Cu") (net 8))
 (segment (start 137.6088 81.6649) (end 138.0055 82.0616) (width 0.25) (layer "B.Cu") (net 8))
 (segment (start 138.0055 82.0616) (end 140.9093 82.0616) (width 0.25) (layer "B.Cu") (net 8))
 (segment (start 148.8 89.4) (end 148.8 91.4) (width 0.7) (layer "F.Cu") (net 6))
 (segment (start 148.9 89.3) (end 148.8 89.4) (width 0.7) (layer "F.Cu") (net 6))
 (segment (start 147.7 93.5801) (end 147.7 94.7) (width 0.7) (layer "F.Cu") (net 6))
 (segment (start 147.7 94.7) (end 142.45 94.7) (width 0.7) (layer "F.Cu") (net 6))
 (segment (start 147.6 93.4801) (end 147.7 93.5801) (width 0.7) (layer "F.Cu") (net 6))
 (segment (start 142.45 94.7) (end 140.95 93.2) (width 0.7) (layer "F.Cu") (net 6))
 (segment (start 138.6 90.3) (end 137.5 90.3) (width 0.7) (layer "F.Cu") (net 6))
 (segment (start 137.085 89.885) (end 137.085 88.245) (width 0.7) (layer "F.Cu") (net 6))
 (segment (start 140.95 92.65) (end 138.6 90.3) (width 0.7) (layer "F.Cu") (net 6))
 (segment (start 140.95 93.2) (end 140.95 92.65) (width 0.25) (layer "F.Cu") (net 6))
 (segment (start 148.8 91.4) (end 147.6 92.6) (width 0.7) (layer "F.Cu") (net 6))
 (segment (start 147.6 92.6) (end 147.6 93.4801) (width 0.7) (layer "F.Cu") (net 6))
 (segment (start 137.5 90.3) (end 137.085 89.885) (width 0.7) (layer "F.Cu") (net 6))
 (segment (start 137.7 93.2) (end 139.05 93.2) (width 0.25) (layer "F.Cu") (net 4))
 (segment (start 134.545 90.045) (end 137.7 93.2) (width 0.25) (layer "F.Cu") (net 4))
 (segment (start 134.545 88.245) (end 134.545 90.045) (width 0.25) (layer "F.Cu") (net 4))
 (segment (start 129.0891 83.0524) (end 129.0891 86.4766) (width 0.25) (layer "F.Cu") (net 9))
 (segment (start 130.1742 81.9673) (end 129.0891 83.0524) (width 0.25) (layer "F.Cu") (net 9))
 (segment (start 135.815 82.8096) (end 134.9727 81.9673) (width 0.25) (layer "F.Cu") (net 9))
 (segment (start 129.0891 86.4766) (end 130.2 87.5875) (width 0.25) (layer "F.Cu") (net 9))
 (segment (start 134.9727 81.9673) (end 130.1742 81.9673) (width 0.25) (layer "F.Cu") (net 9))
 (segment (start 135.815 83.295) (end 135.815 82.8096) (width 0.25) (layer "F.Cu") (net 9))
 (segment (start 136.5875 79) (end 136.6 79.0125) (width 0.25) (layer "F.Cu") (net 7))
 (segment (start 131.5 79) (end 136.5875 79) (width 0.25) (layer "F.Cu") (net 7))
 (segment (start 138.355 83.295) (end 138.355 80.7675) (width 0.25) (layer "F.Cu") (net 7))
 (segment (start 138.355 80.7675) (end 136.6 79.0125) (width 0.25) (layer "F.Cu") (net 7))
 (segment (start 133.55 92.4562) (end 135.3401 92.4562) (width 0.7) (layer "F.Cu") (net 5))
 (segment (start 137.0232 91.4232) (end 135.815 90.215) (width 0.7) (layer "F.Cu") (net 5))
 (segment (start 133.55 98.7233) (end 137.7233 98.7233) (width 0.7) (layer "F.Cu") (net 5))
 (segment (start 133.55 92.8) (end 133.55 92.4562) (width 0.25) (layer "F.Cu") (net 5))
 (segment (start 133.55 92.4562) (end 133.55 92.2458) (width 0.25) (layer "F.Cu") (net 5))
 (segment (start 135.815 90.215) (end 135.815 88.245) (width 0.7) (layer "F.Cu") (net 5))
 (segment (start 137.7233 98.7233) (end 140.5 101.5) (width 0.7) (layer "F.Cu") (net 5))
 (segment (start 140.5 101.5) (end 140.5 102.5) (width 0.7) (layer "F.Cu") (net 5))
 (segment (start 130.7167 89.4125) (end 130.2 89.4125) (width 0.25) (layer "F.Cu") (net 5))
 (segment (start 133.55 92.8) (end 133.55 98.7233) (width 0.7) (layer "F.Cu") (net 5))
 (segment (start 138.1411 91.4232) (end 137.0232 91.4232) (width 0.7) (layer "F.Cu") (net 5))
 (segment (start 133.55 92.2458) (end 130.7167 89.4125) (width 0.25) (layer "F.Cu") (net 5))
 (segment (start 140.5 102.5) (end 139.6 103.4) (width 0.7) (layer "F.Cu") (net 5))
 (via (at 138.1411 91.4232) (size 0.8) (drill 0.4) (layers "F.Cu" "B.Cu") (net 5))
 (via (at 135.3401 92.4562) (size 0.8) (drill 0.4) (layers "F.Cu" "B.Cu") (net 5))
 (segment (start 136.3731 91.4232) (end 138.1411 91.4232) (width 0.7) (layer "B.Cu") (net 5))
 (segment (start 135.3401 92.4562) (end 136.3731 91.4232) (width 0.7) (layer "B.Cu") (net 5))
 (segment (start 149.9 80.1125) (end 148.4125 80.1125) (width 0.7) (layer "F.Cu") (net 11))
 (segment (start 143.15 76.9767) (end 143.9 76.2267) (width 0.25) (layer "F.Cu") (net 11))
 (segment (start 131.5 77.175) (end 133.775 74.9) (width 0.25) (layer "F.Cu") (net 11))
 (segment (start 143.9 75.6) (end 143.9 74.9) (width 0.25) (layer "F.Cu") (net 11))
 (segment (start 149.9 81.0233) (end 149.9 80.1125) (width 0.7) (layer "F.Cu") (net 11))
 (segment (start 148.8 82.1233) (end 149.9 81.0233) (width 0.7) (layer "F.Cu") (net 11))
 (segment (start 148.8 83) (end 148.8 82.1233) (width 0.7) (layer "F.Cu") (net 11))
 (segment (start 143.15 79.5) (end 143.15 76.9767) (width 0.25) (layer "F.Cu") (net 11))
 (segment (start 143.9 74.9) (end 143.9 76.2267) (width 0.25) (layer "F.Cu") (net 11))
 (segment (start 133.775 74.9) (end 143.9 74.9) (width 0.25) (layer "F.Cu") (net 11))
 (segment (start 148.4125 80.1125) (end 143.9 75.6) (width 0.7) (layer "F.Cu") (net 11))
 (segment (start 150.025 78.1625) (end 149.9 78.2875) (width 0.25) (layer "F.Cu") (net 3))
 (segment (start 151.9 78.2625) (end 149.925 78.2625) (width 0.25) (layer "F.Cu") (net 3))
 (segment (start 149.925 78.2625) (end 149.9 78.2875) (width 0.25) (layer "F.Cu") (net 3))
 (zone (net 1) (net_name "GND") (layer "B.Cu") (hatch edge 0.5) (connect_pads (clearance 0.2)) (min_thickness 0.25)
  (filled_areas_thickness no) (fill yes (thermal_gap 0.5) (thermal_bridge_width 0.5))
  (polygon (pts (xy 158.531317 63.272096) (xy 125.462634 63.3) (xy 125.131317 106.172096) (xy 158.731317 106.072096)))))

